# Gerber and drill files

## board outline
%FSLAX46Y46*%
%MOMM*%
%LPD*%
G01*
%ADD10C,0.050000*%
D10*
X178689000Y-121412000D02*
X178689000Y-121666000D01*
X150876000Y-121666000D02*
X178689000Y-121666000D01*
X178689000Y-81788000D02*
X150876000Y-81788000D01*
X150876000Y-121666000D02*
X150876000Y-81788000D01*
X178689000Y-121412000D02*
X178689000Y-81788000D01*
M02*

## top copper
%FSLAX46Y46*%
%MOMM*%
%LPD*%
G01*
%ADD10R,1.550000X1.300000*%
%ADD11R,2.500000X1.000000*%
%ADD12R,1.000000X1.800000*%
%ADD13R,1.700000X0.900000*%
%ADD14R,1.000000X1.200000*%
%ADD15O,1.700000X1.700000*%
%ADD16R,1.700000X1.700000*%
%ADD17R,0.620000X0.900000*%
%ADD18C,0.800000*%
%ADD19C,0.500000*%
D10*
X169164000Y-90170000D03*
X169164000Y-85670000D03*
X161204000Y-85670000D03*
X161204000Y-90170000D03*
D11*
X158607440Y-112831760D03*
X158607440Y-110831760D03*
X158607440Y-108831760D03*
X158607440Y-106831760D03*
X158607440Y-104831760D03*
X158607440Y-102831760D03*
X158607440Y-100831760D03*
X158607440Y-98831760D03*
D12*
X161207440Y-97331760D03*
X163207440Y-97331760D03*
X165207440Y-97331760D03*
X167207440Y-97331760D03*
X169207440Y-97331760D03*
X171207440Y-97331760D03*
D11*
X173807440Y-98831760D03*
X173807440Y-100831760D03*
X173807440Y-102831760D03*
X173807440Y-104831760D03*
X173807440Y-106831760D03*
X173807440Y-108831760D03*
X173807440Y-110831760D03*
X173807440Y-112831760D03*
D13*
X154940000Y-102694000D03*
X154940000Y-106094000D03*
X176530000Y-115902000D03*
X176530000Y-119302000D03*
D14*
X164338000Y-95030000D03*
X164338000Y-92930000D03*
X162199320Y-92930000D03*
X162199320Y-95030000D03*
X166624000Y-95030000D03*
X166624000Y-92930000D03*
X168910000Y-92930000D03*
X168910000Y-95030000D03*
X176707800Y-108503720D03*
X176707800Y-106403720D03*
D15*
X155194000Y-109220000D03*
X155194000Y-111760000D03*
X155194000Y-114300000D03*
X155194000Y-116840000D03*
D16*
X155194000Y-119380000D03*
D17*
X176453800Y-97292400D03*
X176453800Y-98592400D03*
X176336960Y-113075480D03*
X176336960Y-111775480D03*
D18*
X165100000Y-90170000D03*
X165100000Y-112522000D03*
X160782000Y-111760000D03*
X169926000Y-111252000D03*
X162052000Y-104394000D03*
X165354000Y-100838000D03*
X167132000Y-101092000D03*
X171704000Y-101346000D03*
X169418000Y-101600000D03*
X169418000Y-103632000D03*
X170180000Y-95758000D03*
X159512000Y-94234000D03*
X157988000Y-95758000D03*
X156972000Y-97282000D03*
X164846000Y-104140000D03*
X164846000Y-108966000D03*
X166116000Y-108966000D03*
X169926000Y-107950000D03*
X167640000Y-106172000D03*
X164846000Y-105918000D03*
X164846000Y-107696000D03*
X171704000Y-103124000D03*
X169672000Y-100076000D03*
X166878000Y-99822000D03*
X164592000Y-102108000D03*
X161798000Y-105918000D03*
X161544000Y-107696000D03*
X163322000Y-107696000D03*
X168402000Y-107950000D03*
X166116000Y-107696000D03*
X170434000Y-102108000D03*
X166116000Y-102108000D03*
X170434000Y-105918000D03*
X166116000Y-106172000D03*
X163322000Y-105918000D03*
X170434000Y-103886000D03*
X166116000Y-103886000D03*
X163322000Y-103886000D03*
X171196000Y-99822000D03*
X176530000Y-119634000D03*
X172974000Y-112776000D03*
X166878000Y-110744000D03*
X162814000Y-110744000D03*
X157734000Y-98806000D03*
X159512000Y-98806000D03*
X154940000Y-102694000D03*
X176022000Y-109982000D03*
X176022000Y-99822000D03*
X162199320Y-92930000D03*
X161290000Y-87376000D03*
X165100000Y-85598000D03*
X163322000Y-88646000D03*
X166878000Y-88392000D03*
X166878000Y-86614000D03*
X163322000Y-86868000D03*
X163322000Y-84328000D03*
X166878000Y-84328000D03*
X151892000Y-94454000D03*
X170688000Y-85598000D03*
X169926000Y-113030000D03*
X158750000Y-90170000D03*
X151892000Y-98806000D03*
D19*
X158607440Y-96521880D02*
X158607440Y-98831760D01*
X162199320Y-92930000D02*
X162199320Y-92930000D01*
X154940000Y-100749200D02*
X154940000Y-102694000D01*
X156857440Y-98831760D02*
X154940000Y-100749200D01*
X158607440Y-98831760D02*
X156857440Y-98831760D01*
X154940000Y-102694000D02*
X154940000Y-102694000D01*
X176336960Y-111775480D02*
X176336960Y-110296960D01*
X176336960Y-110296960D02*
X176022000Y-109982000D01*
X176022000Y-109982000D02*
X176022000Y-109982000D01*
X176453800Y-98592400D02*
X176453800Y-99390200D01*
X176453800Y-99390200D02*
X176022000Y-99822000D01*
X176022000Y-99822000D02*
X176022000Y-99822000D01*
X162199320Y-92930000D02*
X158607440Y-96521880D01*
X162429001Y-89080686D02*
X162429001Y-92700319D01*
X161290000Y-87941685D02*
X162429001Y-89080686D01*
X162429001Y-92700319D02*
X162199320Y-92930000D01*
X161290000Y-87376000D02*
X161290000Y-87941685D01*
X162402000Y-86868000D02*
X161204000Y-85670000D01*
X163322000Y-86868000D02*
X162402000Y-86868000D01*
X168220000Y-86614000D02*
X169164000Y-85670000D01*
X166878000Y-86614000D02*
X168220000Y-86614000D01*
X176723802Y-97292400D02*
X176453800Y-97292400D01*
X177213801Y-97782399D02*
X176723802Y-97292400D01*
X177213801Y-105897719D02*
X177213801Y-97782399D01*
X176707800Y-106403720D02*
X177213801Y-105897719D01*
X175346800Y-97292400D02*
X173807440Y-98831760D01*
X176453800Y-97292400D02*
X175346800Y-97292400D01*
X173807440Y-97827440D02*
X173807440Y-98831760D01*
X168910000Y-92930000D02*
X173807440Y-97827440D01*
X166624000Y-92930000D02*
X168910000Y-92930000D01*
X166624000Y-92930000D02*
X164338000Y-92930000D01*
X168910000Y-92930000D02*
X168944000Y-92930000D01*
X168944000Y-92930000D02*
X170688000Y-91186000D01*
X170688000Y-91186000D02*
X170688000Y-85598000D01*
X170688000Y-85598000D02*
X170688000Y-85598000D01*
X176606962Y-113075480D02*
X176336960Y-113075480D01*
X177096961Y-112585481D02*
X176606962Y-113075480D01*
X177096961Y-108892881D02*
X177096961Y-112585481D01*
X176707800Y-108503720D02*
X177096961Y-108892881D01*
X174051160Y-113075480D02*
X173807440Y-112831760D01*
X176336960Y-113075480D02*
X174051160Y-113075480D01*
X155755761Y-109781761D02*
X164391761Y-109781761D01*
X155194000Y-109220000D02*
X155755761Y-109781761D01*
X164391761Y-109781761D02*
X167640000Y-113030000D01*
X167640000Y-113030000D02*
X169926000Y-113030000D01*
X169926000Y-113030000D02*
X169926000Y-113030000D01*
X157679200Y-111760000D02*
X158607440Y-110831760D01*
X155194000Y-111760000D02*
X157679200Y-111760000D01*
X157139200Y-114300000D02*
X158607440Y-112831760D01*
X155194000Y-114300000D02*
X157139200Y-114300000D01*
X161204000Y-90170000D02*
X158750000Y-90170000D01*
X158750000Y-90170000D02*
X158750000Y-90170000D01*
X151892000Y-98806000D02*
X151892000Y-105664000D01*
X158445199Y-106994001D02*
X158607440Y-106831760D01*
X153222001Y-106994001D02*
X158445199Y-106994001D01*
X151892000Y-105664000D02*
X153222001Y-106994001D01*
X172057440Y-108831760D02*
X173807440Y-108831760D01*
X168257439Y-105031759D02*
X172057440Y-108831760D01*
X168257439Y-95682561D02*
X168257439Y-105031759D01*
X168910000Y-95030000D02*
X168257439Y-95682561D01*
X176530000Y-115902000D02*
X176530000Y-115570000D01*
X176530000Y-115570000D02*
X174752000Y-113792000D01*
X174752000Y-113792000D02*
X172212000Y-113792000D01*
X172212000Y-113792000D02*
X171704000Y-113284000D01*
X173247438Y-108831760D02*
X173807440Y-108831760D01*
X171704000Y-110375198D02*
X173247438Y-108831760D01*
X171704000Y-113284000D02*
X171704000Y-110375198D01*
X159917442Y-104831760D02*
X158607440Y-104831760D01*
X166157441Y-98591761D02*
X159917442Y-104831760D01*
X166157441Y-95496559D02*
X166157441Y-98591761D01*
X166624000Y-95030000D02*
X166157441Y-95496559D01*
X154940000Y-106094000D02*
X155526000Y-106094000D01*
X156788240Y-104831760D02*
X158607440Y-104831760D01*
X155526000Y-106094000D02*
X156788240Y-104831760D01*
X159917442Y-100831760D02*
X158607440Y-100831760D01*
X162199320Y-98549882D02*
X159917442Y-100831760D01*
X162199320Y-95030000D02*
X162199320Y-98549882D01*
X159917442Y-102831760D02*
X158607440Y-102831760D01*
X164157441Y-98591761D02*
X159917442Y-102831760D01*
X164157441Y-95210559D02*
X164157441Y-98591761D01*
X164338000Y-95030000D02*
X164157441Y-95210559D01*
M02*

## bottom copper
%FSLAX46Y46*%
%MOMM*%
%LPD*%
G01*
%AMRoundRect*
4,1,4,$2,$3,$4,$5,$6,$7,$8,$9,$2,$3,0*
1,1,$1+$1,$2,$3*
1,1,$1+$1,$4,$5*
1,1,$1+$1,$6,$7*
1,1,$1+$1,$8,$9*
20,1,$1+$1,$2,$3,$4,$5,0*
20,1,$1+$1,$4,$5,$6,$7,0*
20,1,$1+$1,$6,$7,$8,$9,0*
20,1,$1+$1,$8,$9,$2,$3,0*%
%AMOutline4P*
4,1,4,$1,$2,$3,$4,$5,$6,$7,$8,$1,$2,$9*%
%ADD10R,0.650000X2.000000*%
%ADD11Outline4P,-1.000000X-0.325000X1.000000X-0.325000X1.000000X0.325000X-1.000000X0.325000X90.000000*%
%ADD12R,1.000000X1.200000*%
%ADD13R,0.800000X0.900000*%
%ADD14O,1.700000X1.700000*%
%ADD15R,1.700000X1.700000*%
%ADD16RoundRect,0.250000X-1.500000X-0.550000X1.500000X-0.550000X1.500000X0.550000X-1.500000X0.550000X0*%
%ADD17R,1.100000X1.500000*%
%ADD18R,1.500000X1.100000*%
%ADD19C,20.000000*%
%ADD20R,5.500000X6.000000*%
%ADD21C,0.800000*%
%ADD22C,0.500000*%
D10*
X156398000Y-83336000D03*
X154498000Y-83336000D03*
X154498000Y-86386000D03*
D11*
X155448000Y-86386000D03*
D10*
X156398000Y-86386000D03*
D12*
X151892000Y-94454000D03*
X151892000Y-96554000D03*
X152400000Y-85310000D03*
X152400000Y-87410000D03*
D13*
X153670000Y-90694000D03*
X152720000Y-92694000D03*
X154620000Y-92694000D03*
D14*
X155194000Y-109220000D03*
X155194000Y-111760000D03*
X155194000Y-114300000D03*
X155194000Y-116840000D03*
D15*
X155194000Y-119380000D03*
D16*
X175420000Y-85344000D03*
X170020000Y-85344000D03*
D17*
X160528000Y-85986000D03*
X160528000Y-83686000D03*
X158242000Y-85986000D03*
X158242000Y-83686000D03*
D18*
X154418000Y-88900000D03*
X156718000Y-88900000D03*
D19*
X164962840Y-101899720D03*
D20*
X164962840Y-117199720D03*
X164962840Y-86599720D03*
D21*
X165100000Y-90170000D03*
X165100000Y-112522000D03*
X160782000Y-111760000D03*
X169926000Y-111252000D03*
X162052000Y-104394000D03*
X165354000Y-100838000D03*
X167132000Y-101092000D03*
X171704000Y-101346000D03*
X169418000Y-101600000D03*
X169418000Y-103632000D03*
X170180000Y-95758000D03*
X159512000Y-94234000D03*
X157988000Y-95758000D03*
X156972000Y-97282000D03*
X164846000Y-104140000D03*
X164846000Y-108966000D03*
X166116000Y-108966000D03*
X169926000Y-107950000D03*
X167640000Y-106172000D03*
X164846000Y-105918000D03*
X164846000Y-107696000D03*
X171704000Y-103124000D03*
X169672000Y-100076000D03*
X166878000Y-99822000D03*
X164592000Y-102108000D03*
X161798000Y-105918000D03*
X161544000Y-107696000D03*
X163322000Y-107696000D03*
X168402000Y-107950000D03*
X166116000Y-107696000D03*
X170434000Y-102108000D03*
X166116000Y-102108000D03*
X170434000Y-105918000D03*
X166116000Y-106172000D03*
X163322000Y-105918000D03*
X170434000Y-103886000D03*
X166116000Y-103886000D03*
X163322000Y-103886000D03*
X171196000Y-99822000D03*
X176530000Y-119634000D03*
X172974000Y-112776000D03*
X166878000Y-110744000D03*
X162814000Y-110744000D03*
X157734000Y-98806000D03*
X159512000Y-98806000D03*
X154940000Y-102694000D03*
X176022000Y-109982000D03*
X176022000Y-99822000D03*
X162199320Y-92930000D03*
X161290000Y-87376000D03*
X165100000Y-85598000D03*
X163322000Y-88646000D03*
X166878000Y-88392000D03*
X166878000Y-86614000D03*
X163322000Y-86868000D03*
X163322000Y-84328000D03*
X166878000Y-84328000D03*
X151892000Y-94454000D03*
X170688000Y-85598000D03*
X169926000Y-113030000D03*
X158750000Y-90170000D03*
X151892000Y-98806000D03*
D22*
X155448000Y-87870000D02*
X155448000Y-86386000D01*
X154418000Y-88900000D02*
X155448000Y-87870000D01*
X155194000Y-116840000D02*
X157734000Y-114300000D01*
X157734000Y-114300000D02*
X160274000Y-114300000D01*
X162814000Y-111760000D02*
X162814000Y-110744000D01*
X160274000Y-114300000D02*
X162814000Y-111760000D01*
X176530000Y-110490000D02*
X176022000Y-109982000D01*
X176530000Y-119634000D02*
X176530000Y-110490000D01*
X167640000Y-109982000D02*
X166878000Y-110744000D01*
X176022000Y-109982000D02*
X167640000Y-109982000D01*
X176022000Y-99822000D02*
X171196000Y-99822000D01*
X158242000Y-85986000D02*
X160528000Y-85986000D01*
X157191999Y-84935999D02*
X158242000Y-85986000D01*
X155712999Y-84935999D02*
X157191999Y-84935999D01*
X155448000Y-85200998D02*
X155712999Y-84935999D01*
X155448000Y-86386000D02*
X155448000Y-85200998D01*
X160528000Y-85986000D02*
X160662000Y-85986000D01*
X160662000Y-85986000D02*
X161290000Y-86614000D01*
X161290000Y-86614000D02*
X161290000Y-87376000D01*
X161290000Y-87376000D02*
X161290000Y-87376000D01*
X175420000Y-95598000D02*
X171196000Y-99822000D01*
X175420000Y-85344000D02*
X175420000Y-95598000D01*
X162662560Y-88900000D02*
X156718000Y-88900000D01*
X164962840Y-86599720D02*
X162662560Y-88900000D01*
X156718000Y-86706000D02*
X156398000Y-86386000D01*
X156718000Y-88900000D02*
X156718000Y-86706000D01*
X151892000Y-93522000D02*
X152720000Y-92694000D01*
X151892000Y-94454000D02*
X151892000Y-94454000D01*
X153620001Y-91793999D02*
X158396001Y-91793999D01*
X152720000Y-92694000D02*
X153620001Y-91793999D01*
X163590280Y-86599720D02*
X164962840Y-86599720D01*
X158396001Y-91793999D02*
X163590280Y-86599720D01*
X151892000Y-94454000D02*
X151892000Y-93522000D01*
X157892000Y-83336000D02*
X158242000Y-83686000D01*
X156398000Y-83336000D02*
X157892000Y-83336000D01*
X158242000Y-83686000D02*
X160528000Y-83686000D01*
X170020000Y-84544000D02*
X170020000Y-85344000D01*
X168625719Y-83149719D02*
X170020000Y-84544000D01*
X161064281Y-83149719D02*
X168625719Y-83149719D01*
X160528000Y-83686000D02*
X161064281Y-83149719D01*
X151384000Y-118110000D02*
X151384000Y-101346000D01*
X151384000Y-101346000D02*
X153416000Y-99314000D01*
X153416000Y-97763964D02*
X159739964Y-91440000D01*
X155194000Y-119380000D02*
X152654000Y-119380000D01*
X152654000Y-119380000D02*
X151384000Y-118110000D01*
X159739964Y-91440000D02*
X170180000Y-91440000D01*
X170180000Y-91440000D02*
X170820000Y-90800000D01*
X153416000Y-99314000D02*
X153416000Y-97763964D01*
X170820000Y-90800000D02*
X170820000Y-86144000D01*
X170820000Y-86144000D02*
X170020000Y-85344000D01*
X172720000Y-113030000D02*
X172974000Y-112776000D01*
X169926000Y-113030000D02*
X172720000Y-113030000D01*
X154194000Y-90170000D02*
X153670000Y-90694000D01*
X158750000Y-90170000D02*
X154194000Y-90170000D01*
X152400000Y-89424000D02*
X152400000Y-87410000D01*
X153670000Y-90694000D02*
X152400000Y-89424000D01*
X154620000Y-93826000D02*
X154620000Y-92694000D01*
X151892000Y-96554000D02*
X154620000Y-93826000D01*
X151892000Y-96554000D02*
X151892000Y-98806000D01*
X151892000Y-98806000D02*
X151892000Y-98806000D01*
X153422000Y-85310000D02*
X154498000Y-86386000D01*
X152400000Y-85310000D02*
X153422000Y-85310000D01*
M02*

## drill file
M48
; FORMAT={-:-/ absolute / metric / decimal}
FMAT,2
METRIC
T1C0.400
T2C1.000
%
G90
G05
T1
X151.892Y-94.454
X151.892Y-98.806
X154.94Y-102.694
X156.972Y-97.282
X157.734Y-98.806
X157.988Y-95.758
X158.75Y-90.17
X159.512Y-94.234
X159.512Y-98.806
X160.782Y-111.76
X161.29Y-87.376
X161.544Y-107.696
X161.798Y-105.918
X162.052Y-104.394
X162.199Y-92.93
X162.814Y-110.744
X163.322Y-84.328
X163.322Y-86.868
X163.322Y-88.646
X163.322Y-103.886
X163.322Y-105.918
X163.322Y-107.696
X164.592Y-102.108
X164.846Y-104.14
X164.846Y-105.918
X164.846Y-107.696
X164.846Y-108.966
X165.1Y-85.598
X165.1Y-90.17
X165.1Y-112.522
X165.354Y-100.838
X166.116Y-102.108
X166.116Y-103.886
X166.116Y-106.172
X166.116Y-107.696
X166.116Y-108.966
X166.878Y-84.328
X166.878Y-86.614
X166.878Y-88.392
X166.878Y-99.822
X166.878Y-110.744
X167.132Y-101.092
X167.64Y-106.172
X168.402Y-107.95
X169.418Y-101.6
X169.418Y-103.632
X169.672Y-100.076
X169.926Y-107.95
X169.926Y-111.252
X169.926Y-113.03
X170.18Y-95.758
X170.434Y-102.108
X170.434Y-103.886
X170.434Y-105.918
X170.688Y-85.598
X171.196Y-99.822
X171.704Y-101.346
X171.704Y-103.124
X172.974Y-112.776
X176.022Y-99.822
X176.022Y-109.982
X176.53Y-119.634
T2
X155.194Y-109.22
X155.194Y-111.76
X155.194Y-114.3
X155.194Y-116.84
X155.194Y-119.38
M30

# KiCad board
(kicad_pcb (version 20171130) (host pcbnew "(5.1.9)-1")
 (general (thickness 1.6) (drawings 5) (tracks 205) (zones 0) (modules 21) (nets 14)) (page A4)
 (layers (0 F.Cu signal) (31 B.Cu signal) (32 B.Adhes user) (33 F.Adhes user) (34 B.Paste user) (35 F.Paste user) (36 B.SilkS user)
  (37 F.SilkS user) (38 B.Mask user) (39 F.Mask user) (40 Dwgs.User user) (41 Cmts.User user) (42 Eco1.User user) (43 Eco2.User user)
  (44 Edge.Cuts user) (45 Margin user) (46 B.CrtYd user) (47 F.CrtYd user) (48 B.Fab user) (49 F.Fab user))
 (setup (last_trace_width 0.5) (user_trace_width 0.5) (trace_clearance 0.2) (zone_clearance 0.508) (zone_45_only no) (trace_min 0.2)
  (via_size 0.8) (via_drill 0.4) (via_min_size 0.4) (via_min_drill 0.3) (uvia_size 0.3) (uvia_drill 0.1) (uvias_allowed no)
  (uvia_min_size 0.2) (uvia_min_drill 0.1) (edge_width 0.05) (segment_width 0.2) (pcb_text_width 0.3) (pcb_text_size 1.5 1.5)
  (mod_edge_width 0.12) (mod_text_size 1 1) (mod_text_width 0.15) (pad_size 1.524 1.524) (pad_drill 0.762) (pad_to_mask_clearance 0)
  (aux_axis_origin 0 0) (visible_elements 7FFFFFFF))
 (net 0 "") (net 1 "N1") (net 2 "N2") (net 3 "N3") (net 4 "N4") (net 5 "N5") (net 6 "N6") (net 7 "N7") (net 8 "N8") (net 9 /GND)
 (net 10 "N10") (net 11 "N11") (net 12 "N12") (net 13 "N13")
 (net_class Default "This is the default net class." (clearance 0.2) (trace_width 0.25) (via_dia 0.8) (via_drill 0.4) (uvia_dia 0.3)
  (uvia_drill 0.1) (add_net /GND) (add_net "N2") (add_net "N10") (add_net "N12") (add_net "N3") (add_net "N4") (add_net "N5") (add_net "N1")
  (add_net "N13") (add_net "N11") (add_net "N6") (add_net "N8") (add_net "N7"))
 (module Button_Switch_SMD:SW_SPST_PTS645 (layer F.Cu) (at 165.184 87.92)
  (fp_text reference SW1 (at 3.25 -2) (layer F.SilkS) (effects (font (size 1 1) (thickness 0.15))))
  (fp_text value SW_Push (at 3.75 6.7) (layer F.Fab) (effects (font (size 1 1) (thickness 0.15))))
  (pad 2 smd rect (at 3.98 2.25) (size 1.55 1.3) (layers F.Cu F.Paste F.Mask) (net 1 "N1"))
  (pad 1 smd rect (at 3.98 -2.25) (size 1.55 1.3) (layers F.Cu F.Paste F.Mask) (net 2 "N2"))
  (pad 1 smd rect (at -3.98 -2.25) (size 1.55 1.3) (layers F.Cu F.Paste F.Mask) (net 2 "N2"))
  (pad 2 smd rect (at -3.98 2.25) (size 1.55 1.3) (layers F.Cu F.Paste F.Mask) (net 1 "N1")))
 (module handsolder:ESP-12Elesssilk (layer F.Cu) (at 166.20744 109.33176 180)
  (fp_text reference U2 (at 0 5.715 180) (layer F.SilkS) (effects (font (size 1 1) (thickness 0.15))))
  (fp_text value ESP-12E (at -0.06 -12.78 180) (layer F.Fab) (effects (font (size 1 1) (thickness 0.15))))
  (pad 22 smd rect (at 7.6 -3.5 180) (size 2.5 1) (layers F.Cu F.Paste F.Mask) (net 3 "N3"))
  (pad 21 smd rect (at 7.6 -1.5 180) (size 2.5 1) (layers F.Cu F.Paste F.Mask) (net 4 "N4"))
  (pad 20 smd rect (at 7.6 0.5 180) (size 2.5 1) (layers F.Cu F.Paste F.Mask))
  (pad 19 smd rect (at 7.6 2.5 180) (size 2.5 1) (layers F.Cu F.Paste F.Mask) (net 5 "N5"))
  (pad 18 smd rect (at 7.6 4.5 180) (size 2.5 1) (layers F.Cu F.Paste F.Mask) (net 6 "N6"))
  (pad 17 smd rect (at 7.6 6.5 180) (size 2.5 1) (layers F.Cu F.Paste F.Mask) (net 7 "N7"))
  (pad 16 smd rect (at 7.6 8.5 180) (size 2.5 1) (layers F.Cu F.Paste F.Mask) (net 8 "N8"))
  (pad 15 smd rect (at 7.6 10.5 180) (size 2.5 1) (layers F.Cu F.Paste F.Mask) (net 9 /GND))
  (pad 14 smd rect (at 5 12 180) (size 1 1.8) (layers F.Cu F.Paste F.Mask))
  (pad 13 smd rect (at 3 12 180) (size 1 1.8) (layers F.Cu F.Paste F.Mask))
  (pad 12 smd rect (at 1 12 180) (size 1 1.8) (layers F.Cu F.Paste F.Mask))
  (pad 11 smd rect (at -1 12 180) (size 1 1.8) (layers F.Cu F.Paste F.Mask))
  (pad 10 smd rect (at -3 12 180) (size 1 1.8) (layers F.Cu F.Paste F.Mask))
  (pad 9 smd rect (at -5 12 180) (size 1 1.8) (layers F.Cu F.Paste F.Mask))
  (pad 8 smd rect (at -7.6 10.5 180) (size 2.5 1) (layers F.Cu F.Paste F.Mask) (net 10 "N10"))
  (pad 7 smd rect (at -7.6 8.5 180) (size 2.5 1) (layers F.Cu F.Paste F.Mask))
  (pad 6 smd rect (at -7.6 6.5 180) (size 2.5 1) (layers F.Cu F.Paste F.Mask))
  (pad 5 smd rect (at -7.6 4.5 180) (size 2.5 1) (layers F.Cu F.Paste F.Mask))
  (pad 4 smd rect (at -7.6 2.5 180) (size 2.5 1) (layers F.Cu F.Paste F.Mask))
  (pad 3 smd rect (at -7.6 0.5 180) (size 2.5 1) (layers F.Cu F.Paste F.Mask) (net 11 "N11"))
  (pad 2 smd rect (at -7.6 -1.5 180) (size 2.5 1) (layers F.Cu F.Paste F.Mask))
  (pad 1 smd rect (at -7.6 -3.5 180) (size 2.5 1) (layers F.Cu F.Paste F.Mask) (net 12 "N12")))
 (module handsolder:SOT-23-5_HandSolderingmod (layer B.Cu) (at 155.448 84.836 90)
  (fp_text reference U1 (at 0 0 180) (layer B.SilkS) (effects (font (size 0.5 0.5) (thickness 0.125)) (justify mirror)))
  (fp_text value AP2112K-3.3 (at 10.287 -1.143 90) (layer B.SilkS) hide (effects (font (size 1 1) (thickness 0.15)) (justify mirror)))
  (pad 5 smd rect (at 1.5 0.95 90) (size 2 0.65) (layers B.Cu B.Paste B.Mask) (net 10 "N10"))
  (pad 4 smd rect (at 1.5 -0.95 90) (size 2 0.65) (layers B.Cu B.Paste B.Mask))
  (pad 3 smd rect (at -1.55 -0.95 90) (size 2 0.65) (layers B.Cu B.Paste B.Mask) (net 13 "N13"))
  (pad 2 smd trapezoid (at -1.55 0 90) (size 2 0.65) (layers B.Cu B.Paste B.Mask) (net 9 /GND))
  (pad 1 smd rect (at -1.55 0.95 90) (size 2 0.65) (layers B.Cu B.Paste B.Mask) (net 2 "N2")))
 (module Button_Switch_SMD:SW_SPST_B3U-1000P (layer F.Cu) (at 154.94 104.394 90)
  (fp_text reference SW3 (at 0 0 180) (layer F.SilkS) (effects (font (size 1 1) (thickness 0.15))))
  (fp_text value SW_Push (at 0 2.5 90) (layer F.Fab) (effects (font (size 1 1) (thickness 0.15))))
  (pad 2 smd rect (at 1.7 0 90) (size 0.9 1.7) (layers F.Cu F.Paste F.Mask) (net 9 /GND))
  (pad 1 smd rect (at -1.7 0 90) (size 0.9 1.7) (layers F.Cu F.Paste F.Mask) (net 6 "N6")))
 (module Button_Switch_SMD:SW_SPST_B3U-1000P (layer F.Cu) (at 176.53 117.602 90)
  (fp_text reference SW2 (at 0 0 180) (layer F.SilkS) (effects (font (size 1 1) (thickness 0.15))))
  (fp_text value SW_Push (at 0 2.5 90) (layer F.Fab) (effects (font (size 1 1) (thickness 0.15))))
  (pad 2 smd rect (at 1.7 0 90) (size 0.9 1.7) (layers F.Cu F.Paste F.Mask) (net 11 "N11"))
  (pad 1 smd rect (at -1.7 0 90) (size 0.9 1.7) (layers F.Cu F.Paste F.Mask) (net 9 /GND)))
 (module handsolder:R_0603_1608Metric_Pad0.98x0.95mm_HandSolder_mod (layer F.Cu) (at 164.338 93.98 270)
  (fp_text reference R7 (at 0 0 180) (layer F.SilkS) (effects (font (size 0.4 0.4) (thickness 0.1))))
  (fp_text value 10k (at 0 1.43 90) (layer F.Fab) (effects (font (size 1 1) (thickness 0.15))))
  (pad 2 smd rect (at 1.05 0 270) (size 1.2 1) (layers F.Cu F.Paste F.Mask) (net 7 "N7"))
  (pad 1 smd rect (at -1.05 0 270) (size 1.2 1) (layers F.Cu F.Paste F.Mask) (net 10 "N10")))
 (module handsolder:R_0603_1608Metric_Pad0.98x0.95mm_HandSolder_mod (layer F.Cu) (at 162.19932 93.98 90)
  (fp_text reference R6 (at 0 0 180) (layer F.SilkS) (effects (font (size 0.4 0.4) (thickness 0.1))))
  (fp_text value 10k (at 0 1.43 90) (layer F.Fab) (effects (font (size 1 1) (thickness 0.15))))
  (pad 2 smd rect (at 1.05 0 90) (size 1.2 1) (layers F.Cu F.Paste F.Mask) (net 9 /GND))
  (pad 1 smd rect (at -1.05 0 90) (size 1.2 1) (layers F.Cu F.Paste F.Mask) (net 8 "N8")))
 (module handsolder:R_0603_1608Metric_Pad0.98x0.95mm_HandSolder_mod (layer F.Cu) (at 166.624 93.98 270)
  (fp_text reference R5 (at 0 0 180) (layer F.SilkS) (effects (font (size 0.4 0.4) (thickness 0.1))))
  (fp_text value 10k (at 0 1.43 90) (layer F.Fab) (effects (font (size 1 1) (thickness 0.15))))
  (pad 2 smd rect (at 1.05 0 270) (size 1.2 1) (layers F.Cu F.Paste F.Mask) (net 6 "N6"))
  (pad 1 smd rect (at -1.05 0 270) (size 1.2 1) (layers F.Cu F.Paste F.Mask) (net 10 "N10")))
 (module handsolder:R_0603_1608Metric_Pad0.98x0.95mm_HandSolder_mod (layer F.Cu) (at 168.91 93.98 90)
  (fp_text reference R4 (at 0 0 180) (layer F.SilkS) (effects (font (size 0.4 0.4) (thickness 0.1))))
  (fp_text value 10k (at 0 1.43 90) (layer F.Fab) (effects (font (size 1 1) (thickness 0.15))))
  (pad 2 smd rect (at 1.05 0 90) (size 1.2 1) (layers F.Cu F.Paste F.Mask) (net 10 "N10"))
  (pad 1 smd rect (at -1.05 0 90) (size 1.2 1) (layers F.Cu F.Paste F.Mask) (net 11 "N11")))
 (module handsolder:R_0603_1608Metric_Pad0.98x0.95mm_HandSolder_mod (layer F.Cu) (at 176.7078 107.45372 270)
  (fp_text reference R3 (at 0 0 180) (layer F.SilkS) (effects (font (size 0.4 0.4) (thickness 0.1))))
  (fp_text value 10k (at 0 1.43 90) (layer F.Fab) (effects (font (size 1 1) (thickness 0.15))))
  (pad 2 smd rect (at 1.05 0 270) (size 1.2 1) (layers F.Cu F.Paste F.Mask) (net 12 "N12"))
  (pad 1 smd rect (at -1.05 0 270) (size 1.2 1) (layers F.Cu F.Paste F.Mask) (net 10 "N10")))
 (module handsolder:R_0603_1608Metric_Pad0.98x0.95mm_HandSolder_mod (layer B.Cu) (at 151.892 95.504 90)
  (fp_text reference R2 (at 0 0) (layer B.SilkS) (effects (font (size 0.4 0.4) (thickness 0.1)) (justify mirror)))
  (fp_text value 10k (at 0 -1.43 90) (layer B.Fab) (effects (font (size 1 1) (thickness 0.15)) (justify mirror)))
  (pad 2 smd rect (at 1.05 0 90) (size 1.2 1) (layers B.Cu B.Paste B.Mask) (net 2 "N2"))
  (pad 1 smd rect (at -1.05 0 90) (size 1.2 1) (layers B.Cu B.Paste B.Mask) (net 5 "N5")))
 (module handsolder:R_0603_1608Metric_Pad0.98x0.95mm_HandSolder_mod (layer B.Cu) (at 152.4 86.36 90)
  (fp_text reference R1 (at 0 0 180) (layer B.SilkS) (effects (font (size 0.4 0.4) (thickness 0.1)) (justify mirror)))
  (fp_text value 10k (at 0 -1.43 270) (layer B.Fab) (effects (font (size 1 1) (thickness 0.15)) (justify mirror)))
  (pad 2 smd rect (at 1.05 0 90) (size 1.2 1) (layers B.Cu B.Paste B.Mask) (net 13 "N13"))
  (pad 1 smd rect (at -1.05 0 90) (size 1.2 1) (layers B.Cu B.Paste B.Mask) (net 1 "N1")))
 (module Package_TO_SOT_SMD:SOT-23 (layer B.Cu) (at 153.67 91.694 90)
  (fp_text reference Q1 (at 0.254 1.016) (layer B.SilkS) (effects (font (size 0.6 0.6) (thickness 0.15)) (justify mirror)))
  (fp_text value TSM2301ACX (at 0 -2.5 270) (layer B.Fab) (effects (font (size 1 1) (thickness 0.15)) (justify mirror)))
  (pad 3 smd rect (at 1 0 90) (size 0.9 0.8) (layers B.Cu B.Paste B.Mask) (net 1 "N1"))
  (pad 2 smd rect (at -1 -0.95 90) (size 0.9 0.8) (layers B.Cu B.Paste B.Mask) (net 2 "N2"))
  (pad 1 smd rect (at -1 0.95 90) (size 0.9 0.8) (layers B.Cu B.Paste B.Mask) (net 5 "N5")))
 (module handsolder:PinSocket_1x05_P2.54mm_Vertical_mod (layer F.Cu) (at 155.194 119.38 180)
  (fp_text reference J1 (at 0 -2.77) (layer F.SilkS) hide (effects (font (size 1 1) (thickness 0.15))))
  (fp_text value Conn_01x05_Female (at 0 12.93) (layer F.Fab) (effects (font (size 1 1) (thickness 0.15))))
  (pad 5 thru_hole oval (at 0 10.16 180) (size 1.7 1.7) (drill 1) (layers *.Cu *.Mask) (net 12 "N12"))
  (pad 4 thru_hole oval (at 0 7.62 180) (size 1.7 1.7) (drill 1) (layers *.Cu *.Mask) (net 4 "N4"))
  (pad 3 thru_hole oval (at 0 5.08 180) (size 1.7 1.7) (drill 1) (layers *.Cu *.Mask) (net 3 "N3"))
  (pad 2 thru_hole oval (at 0 2.54 180) (size 1.7 1.7) (drill 1) (layers *.Cu *.Mask) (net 9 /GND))
  (pad 1 thru_hole rect (at 0 0 180) (size 1.7 1.7) (drill 1) (layers *.Cu *.Mask) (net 10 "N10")))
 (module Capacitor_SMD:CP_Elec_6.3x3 (layer B.Cu) (at 172.72 85.344)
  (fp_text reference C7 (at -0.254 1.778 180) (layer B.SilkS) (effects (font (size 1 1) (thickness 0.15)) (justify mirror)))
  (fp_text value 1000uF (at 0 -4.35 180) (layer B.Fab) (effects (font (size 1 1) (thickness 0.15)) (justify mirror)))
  (pad 2 smd roundrect (at 2.7 0) (size 3.5 1.6) (layers B.Cu B.Paste B.Mask) (roundrect_rratio 0.15625) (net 9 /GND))
  (pad 1 smd roundrect (at -2.7 0) (size 3.5 1.6) (layers B.Cu B.Paste B.Mask) (roundrect_rratio 0.15625) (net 10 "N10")))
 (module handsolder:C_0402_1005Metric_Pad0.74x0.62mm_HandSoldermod (layer F.Cu) (at 176.4538 97.9424 90)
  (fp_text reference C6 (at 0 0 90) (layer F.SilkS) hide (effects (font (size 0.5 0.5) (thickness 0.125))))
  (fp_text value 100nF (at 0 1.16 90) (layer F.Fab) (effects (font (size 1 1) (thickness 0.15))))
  (pad 2 smd rect (at 0.65 0 90) (size 0.9 0.62) (layers F.Cu F.Paste F.Mask) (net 10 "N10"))
  (pad 1 smd rect (at -0.65 0 90) (size 0.9 0.62) (layers F.Cu F.Paste F.Mask) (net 9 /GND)))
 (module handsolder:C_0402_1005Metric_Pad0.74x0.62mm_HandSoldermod (layer F.Cu) (at 176.33696 112.42548 270)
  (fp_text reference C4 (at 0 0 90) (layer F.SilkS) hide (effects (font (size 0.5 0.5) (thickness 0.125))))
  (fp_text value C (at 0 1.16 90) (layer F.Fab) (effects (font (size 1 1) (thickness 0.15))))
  (pad 2 smd rect (at 0.65 0 270) (size 0.9 0.62) (layers F.Cu F.Paste F.Mask) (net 12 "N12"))
  (pad 1 smd rect (at -0.65 0 270) (size 0.9 0.62) (layers F.Cu F.Paste F.Mask) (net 9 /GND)))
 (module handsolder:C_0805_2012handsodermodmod (layer B.Cu) (at 160.528 84.836 270)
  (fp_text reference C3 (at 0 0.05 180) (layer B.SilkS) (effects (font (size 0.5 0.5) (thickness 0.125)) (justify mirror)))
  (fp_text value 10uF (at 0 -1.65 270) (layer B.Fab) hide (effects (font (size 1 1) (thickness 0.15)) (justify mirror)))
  (pad 2 smd rect (at 1.15 0 270) (size 1.5 1.1) (layers B.Cu B.Paste B.Mask) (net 9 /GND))
  (pad 1 smd rect (at -1.15 0 270) (size 1.5 1.1) (layers B.Cu B.Paste B.Mask) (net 10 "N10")))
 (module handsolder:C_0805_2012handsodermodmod (layer B.Cu) (at 158.242 84.836 270)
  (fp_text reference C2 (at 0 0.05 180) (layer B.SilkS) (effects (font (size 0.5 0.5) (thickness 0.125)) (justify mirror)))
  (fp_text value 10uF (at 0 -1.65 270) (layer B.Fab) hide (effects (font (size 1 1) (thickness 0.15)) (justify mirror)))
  (pad 2 smd rect (at 1.15 0 270) (size 1.5 1.1) (layers B.Cu B.Paste B.Mask) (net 9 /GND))
  (pad 1 smd rect (at -1.15 0 270) (size 1.5 1.1) (layers B.Cu B.Paste B.Mask) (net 10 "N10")))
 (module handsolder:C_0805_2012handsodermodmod (layer B.Cu) (at 155.568 88.9 180)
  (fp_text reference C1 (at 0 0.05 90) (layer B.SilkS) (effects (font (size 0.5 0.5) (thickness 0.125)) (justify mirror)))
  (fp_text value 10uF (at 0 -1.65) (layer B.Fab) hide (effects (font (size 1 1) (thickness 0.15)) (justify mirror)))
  (pad 2 smd rect (at 1.15 0 180) (size 1.5 1.1) (layers B.Cu B.Paste B.Mask) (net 9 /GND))
  (pad 1 smd rect (at -1.15 0 180) (size 1.5 1.1) (layers B.Cu B.Paste B.Mask) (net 2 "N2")))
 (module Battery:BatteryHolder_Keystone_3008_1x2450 (layer B.Cu) (at 164.96284 101.89972 270)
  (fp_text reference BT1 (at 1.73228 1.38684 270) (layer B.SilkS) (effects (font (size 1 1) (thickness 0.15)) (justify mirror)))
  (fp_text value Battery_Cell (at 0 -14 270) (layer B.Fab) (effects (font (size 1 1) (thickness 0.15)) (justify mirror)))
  (pad 2 smd circle (at 0 0 270) (size 20 20) (layers B.Cu B.Mask) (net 9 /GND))
  (pad 1 smd rect (at 15.3 0 270) (size 6 5.5) (layers B.Cu B.Paste B.Mask) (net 2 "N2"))
  (pad 1 smd rect (at -15.3 0 270) (size 6 5.5) (layers B.Cu B.Paste B.Mask) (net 2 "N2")))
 (gr_line (start 178.689 121.412) (end 178.689 121.666) (layer Edge.Cuts) (width 0.05))
 (gr_line (start 150.876 121.666) (end 178.689 121.666) (layer Edge.Cuts) (width 0.05))
 (gr_line (start 178.689 81.788) (end 150.876 81.788) (layer Edge.Cuts) (width 0.05))
 (gr_line (start 150.876 121.666) (end 150.876 81.788) (layer Edge.Cuts) (width 0.05))
 (gr_line (start 178.689 121.412) (end 178.689 81.788) (layer Edge.Cuts) (width 0.05))
 (via (at 165.1 90.17) (size 0.8) (drill 0.4) (layers F.Cu B.Cu) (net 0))
 (via (at 165.1 112.522) (size 0.8) (drill 0.4) (layers F.Cu B.Cu) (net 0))
 (via (at 160.782 111.76) (size 0.8) (drill 0.4) (layers F.Cu B.Cu) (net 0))
 (via (at 169.926 111.252) (size 0.8) (drill 0.4) (layers F.Cu B.Cu) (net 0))
 (via (at 162.052 104.394) (size 0.8) (drill 0.4) (layers F.Cu B.Cu) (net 9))
 (via (at 165.354 100.838) (size 0.8) (drill 0.4) (layers F.Cu B.Cu) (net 9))
 (via (at 167.132 101.092) (size 0.8) (drill 0.4) (layers F.Cu B.Cu) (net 9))
 (via (at 171.704 101.346) (size 0.8) (drill 0.4) (layers F.Cu B.Cu) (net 9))
 (via (at 169.418 101.6) (size 0.8) (drill 0.4) (layers F.Cu B.Cu) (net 9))
 (via (at 169.418 103.632) (size 0.8) (drill 0.4) (layers F.Cu B.Cu) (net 9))
 (via (at 170.18 95.758) (size 0.8) (drill 0.4) (layers F.Cu B.Cu) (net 9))
 (via (at 159.512 94.234) (size 0.8) (drill 0.4) (layers F.Cu B.Cu) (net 9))
 (via (at 157.988 95.758) (size 0.8) (drill 0.4) (layers F.Cu B.Cu) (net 9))
 (via (at 156.972 97.282) (size 0.8) (drill 0.4) (layers F.Cu B.Cu) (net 9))
 (via (at 164.846 104.14) (size 0.8) (drill 0.4) (layers F.Cu B.Cu) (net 9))
 (via (at 164.846 108.966) (size 0.8) (drill 0.4) (layers F.Cu B.Cu) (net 9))
 (via (at 166.116 108.966) (size 0.8) (drill 0.4) (layers F.Cu B.Cu) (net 9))
 (via (at 169.926 107.95) (size 0.8) (drill 0.4) (layers F.Cu B.Cu) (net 9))
 (via (at 167.64 106.172) (size 0.8) (drill 0.4) (layers F.Cu B.Cu) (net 9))
 (via (at 164.846 105.918) (size 0.8) (drill 0.4) (layers F.Cu B.Cu) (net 9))
 (via (at 164.846 107.696) (size 0.8) (drill 0.4) (layers F.Cu B.Cu) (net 9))
 (via (at 171.704 103.124) (size 0.8) (drill 0.4) (layers F.Cu B.Cu) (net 9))
 (via (at 169.672 100.076) (size 0.8) (drill 0.4) (layers F.Cu B.Cu) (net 9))
 (via (at 166.878 99.822) (size 0.8) (drill 0.4) (layers F.Cu B.Cu) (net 9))
 (via (at 164.592 102.108) (size 0.8) (drill 0.4) (layers F.Cu B.Cu) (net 9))
 (via (at 161.798 105.918) (size 0.8) (drill 0.4) (layers F.Cu B.Cu) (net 9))
 (via (at 161.544 107.696) (size 0.8) (drill 0.4) (layers F.Cu B.Cu) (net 9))
 (via (at 163.322 107.696) (size 0.8) (drill 0.4) (layers F.Cu B.Cu) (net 9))
 (via (at 168.402 107.95) (size 0.8) (drill 0.4) (layers F.Cu B.Cu) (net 9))
 (via (at 166.116 107.696) (size 0.8) (drill 0.4) (layers F.Cu B.Cu) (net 9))
 (via (at 170.434 102.108) (size 0.8) (drill 0.4) (layers F.Cu B.Cu) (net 9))
 (via (at 166.116 102.108) (size 0.8) (drill 0.4) (layers F.Cu B.Cu) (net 9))
 (via (at 170.434 105.918) (size 0.8) (drill 0.4) (layers F.Cu B.Cu) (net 9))
 (via (at 166.116 106.172) (size 0.8) (drill 0.4) (layers F.Cu B.Cu) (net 9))
 (via (at 163.322 105.918) (size 0.8) (drill 0.4) (layers F.Cu B.Cu) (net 9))
 (via (at 170.434 103.886) (size 0.8) (drill 0.4) (layers F.Cu B.Cu) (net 9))
 (via (at 166.116 103.886) (size 0.8) (drill 0.4) (layers F.Cu B.Cu) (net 9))
 (via (at 163.322 103.886) (size 0.8) (drill 0.4) (layers F.Cu B.Cu) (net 9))
 (via (at 171.196 99.822) (size 0.8) (drill 0.4) (layers F.Cu B.Cu) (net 9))
 (via (at 176.53 119.634) (size 0.8) (drill 0.4) (layers F.Cu B.Cu) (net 9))
 (via (at 172.974 112.776) (size 0.8) (drill 0.4) (layers F.Cu B.Cu) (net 12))
 (via (at 166.878 110.744) (size 0.8) (drill 0.4) (layers F.Cu B.Cu) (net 9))
 (via (at 162.814 110.744) (size 0.8) (drill 0.4) (layers F.Cu B.Cu) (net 9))
 (via (at 157.734 98.806) (size 0.8) (drill 0.4) (layers F.Cu B.Cu) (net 9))
 (via (at 159.512 98.806) (size 0.8) (drill 0.4) (layers F.Cu B.Cu) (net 9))
 (segment (start 155.448 87.87) (end 155.448 86.386) (width 0.5) (layer B.Cu) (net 9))
 (segment (start 154.418 88.9) (end 155.448 87.87) (width 0.5) (layer B.Cu) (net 9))
 (segment (start 158.60744 96.52188) (end 158.60744 98.83176) (width 0.5) (layer F.Cu) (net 9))
 (segment (start 162.19932 92.93) (end 162.19932 92.93) (width 0.5) (layer F.Cu) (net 9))
 (segment (start 154.94 100.7492) (end 154.94 102.694) (width 0.5) (layer F.Cu) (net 9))
 (segment (start 156.85744 98.83176) (end 154.94 100.7492) (width 0.5) (layer F.Cu) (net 9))
 (segment (start 158.60744 98.83176) (end 156.85744 98.83176) (width 0.5) (layer F.Cu) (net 9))
 (segment (start 154.94 102.694) (end 154.94 102.694) (width 0.5) (layer F.Cu) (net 9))
 (via (at 154.94 102.694) (size 0.8) (drill 0.4) (layers F.Cu B.Cu) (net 9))
 (segment (start 155.194 116.84) (end 157.734 114.3) (width 0.5) (layer B.Cu) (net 9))
 (segment (start 157.734 114.3) (end 160.274 114.3) (width 0.5) (layer B.Cu) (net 9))
 (segment (start 162.814 111.76) (end 162.814 110.744) (width 0.5) (layer B.Cu) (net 9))
 (segment (start 160.274 114.3) (end 162.814 111.76) (width 0.5) (layer B.Cu) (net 9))
 (segment (start 176.33696 111.77548) (end 176.33696 110.29696) (width 0.5) (layer F.Cu) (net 9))
 (segment (start 176.33696 110.29696) (end 176.022 109.982) (width 0.5) (layer F.Cu) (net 9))
 (segment (start 176.022 109.982) (end 176.022 109.982) (width 0.5) (layer F.Cu) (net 9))
 (via (at 176.022 109.982) (size 0.8) (drill 0.4) (layers F.Cu B.Cu) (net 9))
 (segment (start 176.53 110.49) (end 176.022 109.982) (width 0.5) (layer B.Cu) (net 9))
 (segment (start 176.53 119.634) (end 176.53 110.49) (width 0.5) (layer B.Cu) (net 9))
 (segment (start 167.64 109.982) (end 166.878 110.744) (width 0.5) (layer B.Cu) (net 9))
 (segment (start 176.022 109.982) (end 167.64 109.982) (width 0.5) (layer B.Cu) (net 9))
 (segment (start 176.4538 98.5924) (end 176.4538 99.3902) (width 0.5) (layer F.Cu) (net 9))
 (segment (start 176.4538 99.3902) (end 176.022 99.822) (width 0.5) (layer F.Cu) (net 9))
 (segment (start 176.022 99.822) (end 176.022 99.822) (width 0.5) (layer F.Cu) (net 9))
 (via (at 176.022 99.822) (size 0.8) (drill 0.4) (layers F.Cu B.Cu) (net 9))
 (segment (start 176.022 99.822) (end 171.196 99.822) (width 0.5) (layer B.Cu) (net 9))
 (segment (start 162.19932 92.93) (end 158.60744 96.52188) (width 0.5) (layer F.Cu) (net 9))
 (via (at 162.19932 92.93) (size 0.8) (drill 0.4) (layers F.Cu B.Cu) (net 9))
 (segment (start 158.242 85.986) (end 160.528 85.986) (width 0.5) (layer B.Cu) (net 9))
 (segment (start 157.191999 84.935999) (end 158.242 85.986) (width 0.5) (layer B.Cu) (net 9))
 (segment (start 155.712999 84.935999) (end 157.191999 84.935999) (width 0.5) (layer B.Cu) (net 9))
 (segment (start 155.448 85.200998) (end 155.712999 84.935999) (width 0.5) (layer B.Cu) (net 9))
 (segment (start 155.448 86.386) (end 155.448 85.200998) (width 0.5) (layer B.Cu) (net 9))
 (segment (start 160.528 85.986) (end 160.662 85.986) (width 0.5) (layer B.Cu) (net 9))
 (segment (start 160.662 85.986) (end 161.29 86.614) (width 0.5) (layer B.Cu) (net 9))
 (segment (start 161.29 86.614) (end 161.29 87.376) (width 0.5) (layer B.Cu) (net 9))
 (segment (start 161.29 87.376) (end 161.29 87.376) (width 0.5) (layer B.Cu) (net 9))
 (via (at 161.29 87.376) (size 0.8) (drill 0.4) (layers F.Cu B.Cu) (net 9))
 (segment (start 162.429001 89.080686) (end 162.429001 92.700319) (width 0.5) (layer F.Cu) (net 9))
 (segment (start 161.29 87.941685) (end 162.429001 89.080686) (width 0.5) (layer F.Cu) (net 9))
 (segment (start 162.429001 92.700319) (end 162.19932 92.93) (width 0.5) (layer F.Cu) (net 9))
 (segment (start 161.29 87.376) (end 161.29 87.941685) (width 0.5) (layer F.Cu) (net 9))
 (segment (start 175.42 95.598) (end 171.196 99.822) (width 0.5) (layer B.Cu) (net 9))
 (segment (start 175.42 85.344) (end 175.42 95.598) (width 0.5) (layer B.Cu) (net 9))
 (via (at 165.1 85.598) (size 0.8) (drill 0.4) (layers F.Cu B.Cu) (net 2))
 (via (at 163.322 88.646) (size 0.8) (drill 0.4) (layers F.Cu B.Cu) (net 2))
 (via (at 166.878 88.392) (size 0.8) (drill 0.4) (layers F.Cu B.Cu) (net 2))
 (via (at 166.878 86.614) (size 0.8) (drill 0.4) (layers F.Cu B.Cu) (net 2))
 (via (at 163.322 86.868) (size 0.8) (drill 0.4) (layers F.Cu B.Cu) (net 2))
 (via (at 163.322 84.328) (size 0.8) (drill 0.4) (layers F.Cu B.Cu) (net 2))
 (via (at 166.878 84.328) (size 0.8) (drill 0.4) (layers F.Cu B.Cu) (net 2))
 (segment (start 162.66256 88.9) (end 156.718 88.9) (width 0.5) (layer B.Cu) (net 2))
 (segment (start 164.96284 86.59972) (end 162.66256 88.9) (width 0.5) (layer B.Cu) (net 2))
 (segment (start 156.718 86.706) (end 156.398 86.386) (width 0.5) (layer B.Cu) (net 2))
 (segment (start 156.718 88.9) (end 156.718 86.706) (width 0.5) (layer B.Cu) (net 2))
 (segment (start 162.402 86.868) (end 161.204 85.67) (width 0.5) (layer F.Cu) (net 2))
 (segment (start 163.322 86.868) (end 162.402 86.868) (width 0.5) (layer F.Cu) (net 2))
 (segment (start 168.22 86.614) (end 169.164 85.67) (width 0.5) (layer F.Cu) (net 2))
 (segment (start 166.878 86.614) (end 168.22 86.614) (width 0.5) (layer F.Cu) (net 2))
 (segment (start 151.892 93.522) (end 152.72 92.694) (width 0.5) (layer B.Cu) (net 2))
 (segment (start 151.892 94.454) (end 151.892 94.454) (width 0.5) (layer B.Cu) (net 2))
 (segment (start 153.620001 91.793999) (end 158.396001 91.793999) (width 0.5) (layer B.Cu) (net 2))
 (segment (start 152.72 92.694) (end 153.620001 91.793999) (width 0.5) (layer B.Cu) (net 2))
 (segment (start 163.59028 86.59972) (end 164.96284 86.59972) (width 0.5) (layer B.Cu) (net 2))
 (segment (start 158.396001 91.793999) (end 163.59028 86.59972) (width 0.5) (layer B.Cu) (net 2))
 (segment (start 151.892 94.454) (end 151.892 93.522) (width 0.5) (layer B.Cu) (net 2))
 (via (at 151.892 94.454) (size 0.8) (drill 0.4) (layers F.Cu B.Cu) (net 2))
 (segment (start 157.892 83.336) (end 158.242 83.686) (width 0.5) (layer B.Cu) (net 10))
 (segment (start 156.398 83.336) (end 157.892 83.336) (width 0.5) (layer B.Cu) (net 10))
 (segment (start 158.242 83.686) (end 160.528 83.686) (width 0.5) (layer B.Cu) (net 10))
 (segment (start 170.02 84.544) (end 170.02 85.344) (width 0.5) (layer B.Cu) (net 10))
 (segment (start 168.625719 83.149719) (end 170.02 84.544) (width 0.5) (layer B.Cu) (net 10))
 (segment (start 161.064281 83.149719) (end 168.625719 83.149719) (width 0.5) (layer B.Cu) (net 10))
 (segment (start 160.528 83.686) (end 161.064281 83.149719) (width 0.5) (layer B.Cu) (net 10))
 (segment (start 176.723802 97.2924) (end 176.4538 97.2924) (width 0.5) (layer F.Cu) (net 10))
 (segment (start 177.213801 97.782399) (end 176.723802 97.2924) (width 0.5) (layer F.Cu) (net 10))
 (segment (start 177.213801 105.897719) (end 177.213801 97.782399) (width 0.5) (layer F.Cu) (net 10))
 (segment (start 176.7078 106.40372) (end 177.213801 105.897719) (width 0.5) (layer F.Cu) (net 10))
 (segment (start 175.3468 97.2924) (end 173.80744 98.83176) (width 0.5) (layer F.Cu) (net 10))
 (segment (start 176.4538 97.2924) (end 175.3468 97.2924) (width 0.5) (layer F.Cu) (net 10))
 (segment (start 173.80744 97.82744) (end 173.80744 98.83176) (width 0.5) (layer F.Cu) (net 10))
 (segment (start 168.91 92.93) (end 173.80744 97.82744) (width 0.5) (layer F.Cu) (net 10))
 (segment (start 166.624 92.93) (end 168.91 92.93) (width 0.5) (layer F.Cu) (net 10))
 (segment (start 166.624 92.93) (end 164.338 92.93) (width 0.5) (layer F.Cu) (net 10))
 (segment (start 151.384 118.11) (end 151.384 101.346) (width 0.5) (layer B.Cu) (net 10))
 (segment (start 151.384 101.346) (end 153.416 99.314) (width 0.5) (layer B.Cu) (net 10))
 (segment (start 153.416 97.763964) (end 159.739964 91.44) (width 0.5) (layer B.Cu) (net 10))
 (segment (start 155.194 119.38) (end 152.654 119.38) (width 0.5) (layer B.Cu) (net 10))
 (segment (start 152.654 119.38) (end 151.384 118.11) (width 0.5) (layer B.Cu) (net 10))
 (segment (start 159.739964 91.44) (end 170.18 91.44) (width 0.5) (layer B.Cu) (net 10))
 (segment (start 170.18 91.44) (end 170.82 90.8) (width 0.5) (layer B.Cu) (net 10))
 (segment (start 153.416 99.314) (end 153.416 97.763964) (width 0.5) (layer B.Cu) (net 10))
 (segment (start 170.82 90.8) (end 170.82 86.144) (width 0.5) (layer B.Cu) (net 10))
 (segment (start 170.82 86.144) (end 170.02 85.344) (width 0.5) (layer B.Cu) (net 10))
 (segment (start 168.91 92.93) (end 168.944 92.93) (width 0.5) (layer F.Cu) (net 10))
 (segment (start 168.944 92.93) (end 170.688 91.186) (width 0.5) (layer F.Cu) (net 10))
 (segment (start 170.688 91.186) (end 170.688 85.598) (width 0.5) (layer F.Cu) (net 10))
 (segment (start 170.688 85.598) (end 170.688 85.598) (width 0.5) (layer F.Cu) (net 10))
 (via (at 170.688 85.598) (size 0.8) (drill 0.4) (layers F.Cu B.Cu) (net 10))
 (segment (start 176.606962 113.07548) (end 176.33696 113.07548) (width 0.5) (layer F.Cu) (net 12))
 (segment (start 177.096961 112.585481) (end 176.606962 113.07548) (width 0.5) (layer F.Cu) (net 12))
 (segment (start 177.096961 108.892881) (end 177.096961 112.585481) (width 0.5) (layer F.Cu) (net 12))
 (segment (start 176.7078 108.50372) (end 177.096961 108.892881) (width 0.5) (layer F.Cu) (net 12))
 (segment (start 174.05116 113.07548) (end 173.80744 112.83176) (width 0.5) (layer F.Cu) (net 12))
 (segment (start 176.33696 113.07548) (end 174.05116 113.07548) (width 0.5) (layer F.Cu) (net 12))
 (segment (start 155.755761 109.781761) (end 164.391761 109.781761) (width 0.5) (layer F.Cu) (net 12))
 (segment (start 155.194 109.22) (end 155.755761 109.781761) (width 0.5) (layer F.Cu) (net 12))
 (segment (start 164.391761 109.781761) (end 167.64 113.03) (width 0.5) (layer F.Cu) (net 12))
 (segment (start 167.64 113.03) (end 169.926 113.03) (width 0.5) (layer F.Cu) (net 12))
 (segment (start 169.926 113.03) (end 169.926 113.03) (width 0.5) (layer F.Cu) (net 12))
 (via (at 169.926 113.03) (size 0.8) (drill 0.4) (layers F.Cu B.Cu) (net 12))
 (segment (start 172.72 113.03) (end 172.974 112.776) (width 0.5) (layer B.Cu) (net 12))
 (segment (start 169.926 113.03) (end 172.72 113.03) (width 0.5) (layer B.Cu) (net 12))
 (segment (start 157.6792 111.76) (end 158.60744 110.83176) (width 0.5) (layer F.Cu) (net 4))
 (segment (start 155.194 111.76) (end 157.6792 111.76) (width 0.5) (layer F.Cu) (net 4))
 (segment (start 157.1392 114.3) (end 158.60744 112.83176) (width 0.5) (layer F.Cu) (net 3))
 (segment (start 155.194 114.3) (end 157.1392 114.3) (width 0.5) (layer F.Cu) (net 3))
 (segment (start 161.204 90.17) (end 158.75 90.17) (width 0.5) (layer F.Cu) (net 1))
 (segment (start 158.75 90.17) (end 158.75 90.17) (width 0.5) (layer F.Cu) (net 1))
 (via (at 158.75 90.17) (size 0.8) (drill 0.4) (layers F.Cu B.Cu) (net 1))
 (segment (start 154.194 90.17) (end 153.67 90.694) (width 0.5) (layer B.Cu) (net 1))
 (segment (start 158.75 90.17) (end 154.194 90.17) (width 0.5) (layer B.Cu) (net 1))
 (segment (start 152.4 89.424) (end 152.4 87.41) (width 0.5) (layer B.Cu) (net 1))
 (segment (start 153.67 90.694) (end 152.4 89.424) (width 0.5) (layer B.Cu) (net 1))
 (segment (start 154.62 93.826) (end 154.62 92.694) (width 0.5) (layer B.Cu) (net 5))
 (segment (start 151.892 96.554) (end 154.62 93.826) (width 0.5) (layer B.Cu) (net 5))
 (segment (start 151.892 96.554) (end 151.892 98.806) (width 0.5) (layer B.Cu) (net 5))
 (segment (start 151.892 98.806) (end 151.892 98.806) (width 0.5) (layer B.Cu) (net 5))
 (via (at 151.892 98.806) (size 0.8) (drill 0.4) (layers F.Cu B.Cu) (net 5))
 (segment (start 151.892 98.806) (end 151.892 105.664) (width 0.5) (layer F.Cu) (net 5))
 (segment (start 158.445199 106.994001) (end 158.60744 106.83176) (width 0.5) (layer F.Cu) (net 5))
 (segment (start 153.222001 106.994001) (end 158.445199 106.994001) (width 0.5) (layer F.Cu) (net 5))
 (segment (start 151.892 105.664) (end 153.222001 106.994001) (width 0.5) (layer F.Cu) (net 5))
 (segment (start 153.422 85.31) (end 154.498 86.386) (width 0.5) (layer B.Cu) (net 13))
 (segment (start 152.4 85.31) (end 153.422 85.31) (width 0.5) (layer B.Cu) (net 13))
 (segment (start 172.05744 108.83176) (end 173.80744 108.83176) (width 0.5) (layer F.Cu) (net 11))
 (segment (start 168.257439 105.031759) (end 172.05744 108.83176) (width 0.5) (layer F.Cu) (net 11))
 (segment (start 168.257439 95.682561) (end 168.257439 105.031759) (width 0.5) (layer F.Cu) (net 11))
 (segment (start 168.91 95.03) (end 168.257439 95.682561) (width 0.5) (layer F.Cu) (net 11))
 (segment (start 176.53 115.902) (end 176.53 115.57) (width 0.5) (layer F.Cu) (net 11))
 (segment (start 176.53 115.57) (end 174.752 113.792) (width 0.5) (layer F.Cu) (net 11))
 (segment (start 174.752 113.792) (end 172.212 113.792) (width 0.5) (layer F.Cu) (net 11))
 (segment (start 172.212 113.792) (end 171.704 113.284) (width 0.5) (layer F.Cu) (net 11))
 (segment (start 173.247438 108.83176) (end 173.80744 108.83176) (width 0.5) (layer F.Cu) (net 11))
 (segment (start 171.704 110.375198) (end 173.247438 108.83176) (width 0.5) (layer F.Cu) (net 11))
 (segment (start 171.704 113.284) (end 171.704 110.375198) (width 0.5) (layer F.Cu) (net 11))
 (segment (start 159.917442 104.83176) (end 158.60744 104.83176) (width 0.5) (layer F.Cu) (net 6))
 (segment (start 166.157441 98.591761) (end 159.917442 104.83176) (width 0.5) (layer F.Cu) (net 6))
 (segment (start 166.157441 95.496559) (end 166.157441 98.591761) (width 0.5) (layer F.Cu) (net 6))
 (segment (start 166.624 95.03) (end 166.157441 95.496559) (width 0.5) (layer F.Cu) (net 6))
 (segment (start 154.94 106.094) (end 155.526 106.094) (width 0.5) (layer F.Cu) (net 6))
 (segment (start 156.78824 104.83176) (end 158.60744 104.83176) (width 0.5) (layer F.Cu) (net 6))
 (segment (start 155.526 106.094) (end 156.78824 104.83176) (width 0.5) (layer F.Cu) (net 6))
 (segment (start 159.917442 100.83176) (end 158.60744 100.83176) (width 0.5) (layer F.Cu) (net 8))
 (segment (start 162.19932 98.549882) (end 159.917442 100.83176) (width 0.5) (layer F.Cu) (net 8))
 (segment (start 162.19932 95.03) (end 162.19932 98.549882) (width 0.5) (layer F.Cu) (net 8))
 (segment (start 159.917442 102.83176) (end 158.60744 102.83176) (width 0.5) (layer F.Cu) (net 7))
 (segment (start 164.157441 98.591761) (end 159.917442 102.83176) (width 0.5) (layer F.Cu) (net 7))
 (segment (start 164.157441 95.210559) (end 164.157441 98.591761) (width 0.5) (layer F.Cu) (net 7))
 (segment (start 164.338 95.03) (end 164.157441 95.210559) (width 0.5) (layer F.Cu) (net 7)))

